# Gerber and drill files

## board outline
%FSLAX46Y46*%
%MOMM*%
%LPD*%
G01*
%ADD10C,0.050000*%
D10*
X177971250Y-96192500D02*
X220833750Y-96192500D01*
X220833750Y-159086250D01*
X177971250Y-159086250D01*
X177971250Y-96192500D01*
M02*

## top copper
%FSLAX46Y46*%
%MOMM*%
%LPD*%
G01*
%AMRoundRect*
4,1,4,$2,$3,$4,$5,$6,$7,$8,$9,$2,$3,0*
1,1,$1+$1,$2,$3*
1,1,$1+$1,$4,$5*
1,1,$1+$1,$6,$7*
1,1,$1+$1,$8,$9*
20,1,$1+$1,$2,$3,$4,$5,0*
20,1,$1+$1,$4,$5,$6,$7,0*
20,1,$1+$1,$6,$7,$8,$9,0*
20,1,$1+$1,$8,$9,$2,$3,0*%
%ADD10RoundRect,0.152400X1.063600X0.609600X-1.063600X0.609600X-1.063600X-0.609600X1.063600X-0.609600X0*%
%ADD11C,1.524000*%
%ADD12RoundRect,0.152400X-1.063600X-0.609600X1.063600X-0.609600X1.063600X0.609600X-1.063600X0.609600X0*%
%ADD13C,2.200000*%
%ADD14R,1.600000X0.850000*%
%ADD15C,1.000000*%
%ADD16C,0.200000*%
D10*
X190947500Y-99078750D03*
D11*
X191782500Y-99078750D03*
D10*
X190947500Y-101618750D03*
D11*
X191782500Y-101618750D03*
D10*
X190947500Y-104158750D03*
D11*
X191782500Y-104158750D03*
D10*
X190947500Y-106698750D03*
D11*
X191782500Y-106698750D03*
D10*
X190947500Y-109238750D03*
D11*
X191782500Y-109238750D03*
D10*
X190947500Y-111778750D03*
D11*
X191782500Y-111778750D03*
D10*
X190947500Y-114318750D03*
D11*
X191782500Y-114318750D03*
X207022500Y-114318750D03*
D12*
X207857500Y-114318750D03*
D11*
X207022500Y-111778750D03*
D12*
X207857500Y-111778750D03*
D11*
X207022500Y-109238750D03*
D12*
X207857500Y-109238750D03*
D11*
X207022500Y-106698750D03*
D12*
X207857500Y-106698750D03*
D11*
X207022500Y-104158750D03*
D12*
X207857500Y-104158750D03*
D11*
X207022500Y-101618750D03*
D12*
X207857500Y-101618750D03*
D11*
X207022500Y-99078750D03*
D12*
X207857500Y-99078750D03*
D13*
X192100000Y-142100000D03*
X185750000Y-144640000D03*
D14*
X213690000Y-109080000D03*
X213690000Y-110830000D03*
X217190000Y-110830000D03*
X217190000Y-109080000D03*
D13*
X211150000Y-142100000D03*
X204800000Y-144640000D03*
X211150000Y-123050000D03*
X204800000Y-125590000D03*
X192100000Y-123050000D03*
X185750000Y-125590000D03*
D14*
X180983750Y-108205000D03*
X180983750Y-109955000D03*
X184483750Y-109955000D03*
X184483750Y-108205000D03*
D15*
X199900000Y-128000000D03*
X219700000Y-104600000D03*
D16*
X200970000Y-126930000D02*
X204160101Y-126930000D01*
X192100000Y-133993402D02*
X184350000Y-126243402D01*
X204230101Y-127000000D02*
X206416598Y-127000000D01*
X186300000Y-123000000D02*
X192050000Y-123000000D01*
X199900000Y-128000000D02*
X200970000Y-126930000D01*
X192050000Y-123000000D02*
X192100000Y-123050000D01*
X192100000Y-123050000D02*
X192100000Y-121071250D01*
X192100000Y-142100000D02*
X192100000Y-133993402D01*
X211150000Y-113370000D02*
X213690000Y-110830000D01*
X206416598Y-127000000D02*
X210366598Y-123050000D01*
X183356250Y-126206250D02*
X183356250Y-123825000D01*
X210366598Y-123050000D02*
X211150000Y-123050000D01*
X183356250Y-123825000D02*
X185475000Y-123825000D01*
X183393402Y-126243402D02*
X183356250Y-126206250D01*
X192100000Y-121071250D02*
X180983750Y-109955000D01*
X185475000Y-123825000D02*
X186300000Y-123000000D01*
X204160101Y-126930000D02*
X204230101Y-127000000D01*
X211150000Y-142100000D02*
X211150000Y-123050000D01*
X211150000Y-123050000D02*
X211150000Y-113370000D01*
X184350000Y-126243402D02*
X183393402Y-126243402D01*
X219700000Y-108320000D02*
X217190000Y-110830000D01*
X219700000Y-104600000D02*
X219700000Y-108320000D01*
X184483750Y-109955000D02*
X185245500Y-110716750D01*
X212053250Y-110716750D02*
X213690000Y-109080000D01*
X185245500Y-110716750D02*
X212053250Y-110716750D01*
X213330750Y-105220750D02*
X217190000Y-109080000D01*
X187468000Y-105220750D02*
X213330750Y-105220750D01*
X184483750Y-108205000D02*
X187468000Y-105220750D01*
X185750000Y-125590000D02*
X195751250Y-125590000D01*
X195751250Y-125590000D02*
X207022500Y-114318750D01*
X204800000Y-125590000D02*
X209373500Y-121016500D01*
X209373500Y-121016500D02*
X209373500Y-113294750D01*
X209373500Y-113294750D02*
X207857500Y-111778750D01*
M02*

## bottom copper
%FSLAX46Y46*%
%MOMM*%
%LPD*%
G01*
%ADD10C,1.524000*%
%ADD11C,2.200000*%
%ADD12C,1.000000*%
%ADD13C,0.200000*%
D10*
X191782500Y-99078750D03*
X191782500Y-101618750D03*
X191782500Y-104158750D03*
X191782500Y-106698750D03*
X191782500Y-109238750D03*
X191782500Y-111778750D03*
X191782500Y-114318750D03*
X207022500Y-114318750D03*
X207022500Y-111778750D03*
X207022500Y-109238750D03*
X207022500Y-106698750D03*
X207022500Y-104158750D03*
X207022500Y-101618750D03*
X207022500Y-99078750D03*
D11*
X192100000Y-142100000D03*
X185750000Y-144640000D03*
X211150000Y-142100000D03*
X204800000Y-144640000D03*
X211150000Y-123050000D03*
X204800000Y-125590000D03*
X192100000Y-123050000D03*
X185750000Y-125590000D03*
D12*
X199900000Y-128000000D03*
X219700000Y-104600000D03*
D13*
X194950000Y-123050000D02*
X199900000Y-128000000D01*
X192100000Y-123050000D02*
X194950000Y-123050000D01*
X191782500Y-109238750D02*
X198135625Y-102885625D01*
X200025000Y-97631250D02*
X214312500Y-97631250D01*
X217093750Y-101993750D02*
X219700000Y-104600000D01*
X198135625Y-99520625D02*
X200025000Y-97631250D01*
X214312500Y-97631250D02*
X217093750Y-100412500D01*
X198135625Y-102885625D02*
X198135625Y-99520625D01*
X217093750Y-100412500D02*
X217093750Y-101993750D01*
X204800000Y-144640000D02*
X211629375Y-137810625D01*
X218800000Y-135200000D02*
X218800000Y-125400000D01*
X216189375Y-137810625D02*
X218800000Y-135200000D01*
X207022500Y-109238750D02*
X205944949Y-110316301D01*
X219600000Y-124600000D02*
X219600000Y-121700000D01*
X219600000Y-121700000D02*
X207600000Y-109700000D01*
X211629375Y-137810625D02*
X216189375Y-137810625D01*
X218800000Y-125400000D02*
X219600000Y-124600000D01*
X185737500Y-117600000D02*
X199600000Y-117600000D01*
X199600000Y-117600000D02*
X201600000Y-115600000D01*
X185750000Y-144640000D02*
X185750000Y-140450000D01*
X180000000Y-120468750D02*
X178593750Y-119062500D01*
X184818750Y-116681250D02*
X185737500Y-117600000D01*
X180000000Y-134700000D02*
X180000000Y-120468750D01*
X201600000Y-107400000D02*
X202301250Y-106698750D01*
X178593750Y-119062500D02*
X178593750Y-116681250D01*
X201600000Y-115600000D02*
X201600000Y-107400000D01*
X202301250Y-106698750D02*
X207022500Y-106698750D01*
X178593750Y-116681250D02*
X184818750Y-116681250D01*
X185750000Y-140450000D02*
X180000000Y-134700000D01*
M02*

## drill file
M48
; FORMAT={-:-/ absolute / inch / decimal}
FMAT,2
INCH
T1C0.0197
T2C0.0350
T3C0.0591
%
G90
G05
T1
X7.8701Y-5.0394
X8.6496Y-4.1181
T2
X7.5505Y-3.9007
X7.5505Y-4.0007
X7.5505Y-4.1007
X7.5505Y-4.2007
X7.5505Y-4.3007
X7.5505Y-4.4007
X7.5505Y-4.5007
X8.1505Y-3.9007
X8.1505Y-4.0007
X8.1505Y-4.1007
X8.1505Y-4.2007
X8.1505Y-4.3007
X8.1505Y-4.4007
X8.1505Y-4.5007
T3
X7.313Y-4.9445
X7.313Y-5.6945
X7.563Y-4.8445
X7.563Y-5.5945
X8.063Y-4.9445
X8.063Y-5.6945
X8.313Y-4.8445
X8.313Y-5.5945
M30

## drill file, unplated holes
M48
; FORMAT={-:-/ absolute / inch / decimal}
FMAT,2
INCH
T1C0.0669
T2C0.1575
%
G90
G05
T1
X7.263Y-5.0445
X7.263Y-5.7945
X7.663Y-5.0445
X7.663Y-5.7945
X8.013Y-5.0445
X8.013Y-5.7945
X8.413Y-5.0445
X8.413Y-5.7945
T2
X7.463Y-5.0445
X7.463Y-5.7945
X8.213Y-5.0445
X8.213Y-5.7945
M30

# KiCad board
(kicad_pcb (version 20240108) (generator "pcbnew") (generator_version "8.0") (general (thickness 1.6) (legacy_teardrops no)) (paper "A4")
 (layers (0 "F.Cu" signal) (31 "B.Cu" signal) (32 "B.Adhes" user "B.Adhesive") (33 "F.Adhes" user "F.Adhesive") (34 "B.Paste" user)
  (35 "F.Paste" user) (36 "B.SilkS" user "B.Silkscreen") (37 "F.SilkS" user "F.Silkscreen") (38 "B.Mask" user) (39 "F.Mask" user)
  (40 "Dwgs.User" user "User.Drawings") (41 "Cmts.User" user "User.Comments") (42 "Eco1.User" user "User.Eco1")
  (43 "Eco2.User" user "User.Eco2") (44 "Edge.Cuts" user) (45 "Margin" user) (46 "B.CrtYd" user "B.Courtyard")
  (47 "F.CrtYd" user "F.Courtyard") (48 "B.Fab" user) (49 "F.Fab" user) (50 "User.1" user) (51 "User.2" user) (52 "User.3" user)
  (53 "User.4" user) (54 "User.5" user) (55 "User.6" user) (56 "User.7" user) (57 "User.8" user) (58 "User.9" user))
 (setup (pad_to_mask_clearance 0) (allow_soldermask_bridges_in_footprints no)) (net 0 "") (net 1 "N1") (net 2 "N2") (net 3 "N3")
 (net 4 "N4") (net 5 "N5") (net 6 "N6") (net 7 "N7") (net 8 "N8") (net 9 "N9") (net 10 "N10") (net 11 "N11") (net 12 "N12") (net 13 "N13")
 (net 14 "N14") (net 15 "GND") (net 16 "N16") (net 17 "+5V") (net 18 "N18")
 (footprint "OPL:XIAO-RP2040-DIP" (layer "F.Cu") (at 199.4025 106.69875)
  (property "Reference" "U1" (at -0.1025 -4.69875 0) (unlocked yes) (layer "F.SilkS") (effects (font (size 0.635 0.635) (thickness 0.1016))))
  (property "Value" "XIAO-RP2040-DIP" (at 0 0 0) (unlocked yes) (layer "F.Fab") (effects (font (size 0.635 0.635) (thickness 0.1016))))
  (pad "1" smd roundrect (at -8.455 -7.62 180) (size 2.432 1.524) (layers "F.Cu" "F.Mask") (roundrect_rratio 0.1) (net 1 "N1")
   (thermal_bridge_angle 45))
  (pad "1" thru_hole circle (at -7.62 -7.62 180) (size 1.524 1.524) (drill 0.889) (layers "*.Cu" "*.Mask") (remove_unused_layers no)
   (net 1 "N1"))
  (pad "2" smd roundrect (at -8.455 -5.08 180) (size 2.432 1.524) (layers "F.Cu" "F.Mask") (roundrect_rratio 0.1) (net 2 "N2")
   (thermal_bridge_angle 45))
  (pad "2" thru_hole circle (at -7.62 -5.08 180) (size 1.524 1.524) (drill 0.889) (layers "*.Cu" "*.Mask") (remove_unused_layers no)
   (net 2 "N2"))
  (pad "3" smd roundrect (at -8.455 -2.54 180) (size 2.432 1.524) (layers "F.Cu" "F.Mask") (roundrect_rratio 0.1) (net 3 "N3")
   (thermal_bridge_angle 45))
  (pad "3" thru_hole circle (at -7.62 -2.54 180) (size 1.524 1.524) (drill 0.889) (layers "*.Cu" "*.Mask") (remove_unused_layers no)
   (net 3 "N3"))
  (pad "4" smd roundrect (at -8.455 0 180) (size 2.432 1.524) (layers "F.Cu" "F.Mask") (roundrect_rratio 0.1) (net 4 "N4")
   (thermal_bridge_angle 45))
  (pad "4" thru_hole circle (at -7.62 0 180) (size 1.524 1.524) (drill 0.889) (layers "*.Cu" "*.Mask") (remove_unused_layers no)
   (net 4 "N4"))
  (pad "5" smd roundrect (at -8.455 2.54 180) (size 2.432 1.524) (layers "F.Cu" "F.Mask") (roundrect_rratio 0.1) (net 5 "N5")
   (thermal_bridge_angle 45))
  (pad "5" thru_hole circle (at -7.62 2.54 180) (size 1.524 1.524) (drill 0.889) (layers "*.Cu" "*.Mask") (remove_unused_layers no)
   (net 5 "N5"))
  (pad "6" smd roundrect (at -8.455 5.08 180) (size 2.432 1.524) (layers "F.Cu" "F.Mask") (roundrect_rratio 0.1) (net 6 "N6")
   (thermal_bridge_angle 45))
  (pad "6" thru_hole circle (at -7.62 5.08 180) (size 1.524 1.524) (drill 0.889) (layers "*.Cu" "*.Mask") (remove_unused_layers no)
   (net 6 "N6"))
  (pad "7" smd roundrect (at -8.455 7.62 180) (size 2.432 1.524) (layers "F.Cu" "F.Mask") (roundrect_rratio 0.1) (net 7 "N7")
   (thermal_bridge_angle 45))
  (pad "7" thru_hole circle (at -7.62 7.62 180) (size 1.524 1.524) (drill 0.889) (layers "*.Cu" "*.Mask") (remove_unused_layers no)
   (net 7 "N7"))
  (pad "8" thru_hole circle (at 7.62 7.62) (size 1.524 1.524) (drill 0.889) (layers "*.Cu" "*.Mask") (remove_unused_layers no) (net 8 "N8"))
  (pad "8" smd roundrect (at 8.455 7.62) (size 2.432 1.524) (layers "F.Cu" "F.Mask") (roundrect_rratio 0.1) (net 8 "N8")
   (thermal_bridge_angle 45))
  (pad "9" thru_hole circle (at 7.62 5.08) (size 1.524 1.524) (drill 0.889) (layers "*.Cu" "*.Mask") (remove_unused_layers no) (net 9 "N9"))
  (pad "9" smd roundrect (at 8.455 5.08) (size 2.432 1.524) (layers "F.Cu" "F.Mask") (roundrect_rratio 0.1) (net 9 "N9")
   (thermal_bridge_angle 45))
  (pad "10" thru_hole circle (at 7.62 2.54) (size 1.524 1.524) (drill 0.889) (layers "*.Cu" "*.Mask") (remove_unused_layers no)
   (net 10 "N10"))
  (pad "10" smd roundrect (at 8.455 2.54) (size 2.432 1.524) (layers "F.Cu" "F.Mask") (roundrect_rratio 0.1) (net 10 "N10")
   (thermal_bridge_angle 45))
  (pad "11" thru_hole circle (at 7.62 0) (size 1.524 1.524) (drill 0.889) (layers "*.Cu" "*.Mask") (remove_unused_layers no) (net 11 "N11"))
  (pad "11" smd roundrect (at 8.455 0) (size 2.432 1.524) (layers "F.Cu" "F.Mask") (roundrect_rratio 0.1) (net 11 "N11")
   (thermal_bridge_angle 45))
  (pad "12" thru_hole circle (at 7.62 -2.54) (size 1.524 1.524) (drill 0.889) (layers "*.Cu" "*.Mask") (remove_unused_layers no)
   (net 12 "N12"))
  (pad "12" smd roundrect (at 8.455 -2.54) (size 2.432 1.524) (layers "F.Cu" "F.Mask") (roundrect_rratio 0.1) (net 12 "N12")
   (thermal_bridge_angle 45))
  (pad "13" thru_hole circle (at 7.62 -5.08) (size 1.524 1.524) (drill 0.889) (layers "*.Cu" "*.Mask") (remove_unused_layers no)
   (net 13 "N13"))
  (pad "13" smd roundrect (at 8.455 -5.08) (size 2.432 1.524) (layers "F.Cu" "F.Mask") (roundrect_rratio 0.1) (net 13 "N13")
   (thermal_bridge_angle 45))
  (pad "14" thru_hole circle (at 7.62 -7.62) (size 1.524 1.524) (drill 0.889) (layers "*.Cu" "*.Mask") (remove_unused_layers no)
   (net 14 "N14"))
  (pad "14" smd roundrect (at 8.455 -7.62) (size 2.432 1.524) (layers "F.Cu" "F.Mask") (roundrect_rratio 0.1) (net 14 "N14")
   (thermal_bridge_angle 45)))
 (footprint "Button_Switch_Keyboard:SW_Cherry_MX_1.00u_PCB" (layer "F.Cu") (at 192.1 142.1)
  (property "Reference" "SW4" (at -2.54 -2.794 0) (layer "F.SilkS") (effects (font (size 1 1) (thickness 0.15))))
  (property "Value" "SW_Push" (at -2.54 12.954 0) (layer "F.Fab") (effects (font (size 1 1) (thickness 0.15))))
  (pad "" np_thru_hole circle (at -7.62 5.08) (size 1.7 1.7) (drill 1.7) (layers "*.Cu" "*.Mask"))
  (pad "" np_thru_hole circle (at -2.54 5.08) (size 4 4) (drill 4) (layers "*.Cu" "*.Mask"))
  (pad "" np_thru_hole circle (at 2.54 5.08) (size 1.7 1.7) (drill 1.7) (layers "*.Cu" "*.Mask"))
  (pad "1" thru_hole circle (at 0 0) (size 2.2 2.2) (drill 1.5) (layers "*.Cu" "*.Mask") (remove_unused_layers no) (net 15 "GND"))
  (pad "2" thru_hole circle (at -6.35 2.54) (size 2.2 2.2) (drill 1.5) (layers "*.Cu" "*.Mask") (remove_unused_layers no) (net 11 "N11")))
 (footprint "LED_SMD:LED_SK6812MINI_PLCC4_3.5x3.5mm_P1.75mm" (layer "F.Cu") (at 215.44 109.955)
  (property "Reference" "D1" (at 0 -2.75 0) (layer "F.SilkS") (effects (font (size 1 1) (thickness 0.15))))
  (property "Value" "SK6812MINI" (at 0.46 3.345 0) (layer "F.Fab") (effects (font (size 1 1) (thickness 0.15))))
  (pad "1" smd rect (at -1.75 -0.875) (size 1.6 0.85) (layers "F.Cu" "F.Paste" "F.Mask") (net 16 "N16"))
  (pad "2" smd rect (at -1.75 0.875) (size 1.6 0.85) (layers "F.Cu" "F.Paste" "F.Mask") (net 15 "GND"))
  (pad "3" smd rect (at 1.75 0.875) (size 1.6 0.85) (layers "F.Cu" "F.Paste" "F.Mask") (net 5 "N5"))
  (pad "4" smd rect (at 1.75 -0.875) (size 1.6 0.85) (layers "F.Cu" "F.Paste" "F.Mask") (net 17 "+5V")))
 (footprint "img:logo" (layer "F.Cu") (at 215.554742 100.650524)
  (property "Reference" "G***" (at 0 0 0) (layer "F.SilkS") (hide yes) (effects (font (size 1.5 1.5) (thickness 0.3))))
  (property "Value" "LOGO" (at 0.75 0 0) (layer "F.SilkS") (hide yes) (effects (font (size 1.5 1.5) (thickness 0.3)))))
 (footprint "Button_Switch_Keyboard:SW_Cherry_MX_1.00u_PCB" (layer "F.Cu") (at 211.15 142.1)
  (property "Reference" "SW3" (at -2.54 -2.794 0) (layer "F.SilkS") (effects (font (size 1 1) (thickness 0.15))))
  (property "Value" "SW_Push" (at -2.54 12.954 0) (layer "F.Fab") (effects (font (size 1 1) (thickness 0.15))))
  (pad "" np_thru_hole circle (at -7.62 5.08) (size 1.7 1.7) (drill 1.7) (layers "*.Cu" "*.Mask"))
  (pad "" np_thru_hole circle (at -2.54 5.08) (size 4 4) (drill 4) (layers "*.Cu" "*.Mask"))
  (pad "" np_thru_hole circle (at 2.54 5.08) (size 1.7 1.7) (drill 1.7) (layers "*.Cu" "*.Mask"))
  (pad "1" thru_hole circle (at 0 0) (size 2.2 2.2) (drill 1.5) (layers "*.Cu" "*.Mask") (remove_unused_layers no) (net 15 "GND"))
  (pad "2" thru_hole circle (at -6.35 2.54) (size 2.2 2.2) (drill 1.5) (layers "*.Cu" "*.Mask") (remove_unused_layers no) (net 10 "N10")))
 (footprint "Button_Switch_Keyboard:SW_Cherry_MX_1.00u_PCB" (layer "F.Cu") (at 211.15 123.05)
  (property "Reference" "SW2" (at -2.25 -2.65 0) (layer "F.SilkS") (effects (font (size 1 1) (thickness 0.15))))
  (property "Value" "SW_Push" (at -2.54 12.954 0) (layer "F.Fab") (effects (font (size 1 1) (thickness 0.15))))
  (pad "" np_thru_hole circle (at -7.62 5.08) (size 1.7 1.7) (drill 1.7) (layers "*.Cu" "*.Mask"))
  (pad "" np_thru_hole circle (at -2.54 5.08) (size 4 4) (drill 4) (layers "*.Cu" "*.Mask"))
  (pad "" np_thru_hole circle (at 2.54 5.08) (size 1.7 1.7) (drill 1.7) (layers "*.Cu" "*.Mask"))
  (pad "1" thru_hole circle (at 0 0) (size 2.2 2.2) (drill 1.5) (layers "*.Cu" "*.Mask") (remove_unused_layers no) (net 15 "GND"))
  (pad "2" thru_hole circle (at -6.35 2.54) (size 2.2 2.2) (drill 1.5) (layers "*.Cu" "*.Mask") (remove_unused_layers no) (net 9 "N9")))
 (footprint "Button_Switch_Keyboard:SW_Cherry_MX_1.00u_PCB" (layer "F.Cu") (at 192.1 123.05)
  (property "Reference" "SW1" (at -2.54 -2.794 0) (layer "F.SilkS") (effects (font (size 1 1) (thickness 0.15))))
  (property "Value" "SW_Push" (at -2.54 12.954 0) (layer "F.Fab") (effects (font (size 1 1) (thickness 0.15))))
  (pad "" np_thru_hole circle (at -7.62 5.08) (size 1.7 1.7) (drill 1.7) (layers "*.Cu" "*.Mask"))
  (pad "" np_thru_hole circle (at -2.54 5.08) (size 4 4) (drill 4) (layers "*.Cu" "*.Mask"))
  (pad "" np_thru_hole circle (at 2.54 5.08) (size 1.7 1.7) (drill 1.7) (layers "*.Cu" "*.Mask"))
  (pad "1" thru_hole circle (at 0 0) (size 2.2 2.2) (drill 1.5) (layers "*.Cu" "*.Mask") (remove_unused_layers no) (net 15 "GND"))
  (pad "2" thru_hole circle (at -6.35 2.54) (size 2.2 2.2) (drill 1.5) (layers "*.Cu" "*.Mask") (remove_unused_layers no) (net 8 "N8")))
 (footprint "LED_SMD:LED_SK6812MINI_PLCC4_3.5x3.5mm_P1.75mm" (layer "F.Cu") (at 182.73375 109.08)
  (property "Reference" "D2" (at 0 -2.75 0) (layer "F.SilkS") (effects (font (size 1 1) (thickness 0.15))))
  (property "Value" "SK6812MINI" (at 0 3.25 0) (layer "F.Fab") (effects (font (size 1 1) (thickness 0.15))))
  (pad "1" smd rect (at -1.75 -0.875) (size 1.6 0.85) (layers "F.Cu" "F.Paste" "F.Mask") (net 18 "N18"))
  (pad "2" smd rect (at -1.75 0.875) (size 1.6 0.85) (layers "F.Cu" "F.Paste" "F.Mask") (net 15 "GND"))
  (pad "3" smd rect (at 1.75 0.875) (size 1.6 0.85) (layers "F.Cu" "F.Paste" "F.Mask") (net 16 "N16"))
  (pad "4" smd rect (at 1.75 -0.875) (size 1.6 0.85) (layers "F.Cu" "F.Paste" "F.Mask") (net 17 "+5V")))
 (gr_rect (start 177.97125 96.1925) (end 220.83375 159.08625) (stroke (width 0.05) (type default)) (fill none) (layer "Edge.Cuts"))
 (segment (start 200.97 126.93) (end 204.160101 126.93) (width 0.2) (layer "F.Cu") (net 15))
 (segment (start 192.1 133.993402) (end 184.35 126.243402) (width 0.2) (layer "F.Cu") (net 15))
 (segment (start 204.230101 127) (end 206.416598 127) (width 0.2) (layer "F.Cu") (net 15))
 (segment (start 186.3 123) (end 192.05 123) (width 0.2) (layer "F.Cu") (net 15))
 (segment (start 199.9 128) (end 200.97 126.93) (width 0.2) (layer "F.Cu") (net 15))
 (segment (start 192.05 123) (end 192.1 123.05) (width 0.2) (layer "F.Cu") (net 15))
 (segment (start 192.1 123.05) (end 192.1 121.07125) (width 0.2) (layer "F.Cu") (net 15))
 (segment (start 192.1 142.1) (end 192.1 133.993402) (width 0.2) (layer "F.Cu") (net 15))
 (segment (start 211.15 113.37) (end 213.69 110.83) (width 0.2) (layer "F.Cu") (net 15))
 (segment (start 206.416598 127) (end 210.366598 123.05) (width 0.2) (layer "F.Cu") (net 15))
 (segment (start 183.35625 126.20625) (end 183.35625 123.825) (width 0.2) (layer "F.Cu") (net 15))
 (segment (start 210.366598 123.05) (end 211.15 123.05) (width 0.2) (layer "F.Cu") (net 15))
 (segment (start 183.35625 123.825) (end 185.475 123.825) (width 0.2) (layer "F.Cu") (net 15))
 (segment (start 183.393402 126.243402) (end 183.35625 126.20625) (width 0.2) (layer "F.Cu") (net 15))
 (segment (start 192.1 121.07125) (end 180.98375 109.955) (width 0.2) (layer "F.Cu") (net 15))
 (segment (start 185.475 123.825) (end 186.3 123) (width 0.2) (layer "F.Cu") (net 15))
 (segment (start 204.160101 126.93) (end 204.230101 127) (width 0.2) (layer "F.Cu") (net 15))
 (segment (start 211.15 142.1) (end 211.15 123.05) (width 0.2) (layer "F.Cu") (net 15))
 (segment (start 211.15 123.05) (end 211.15 113.37) (width 0.2) (layer "F.Cu") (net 15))
 (segment (start 184.35 126.243402) (end 183.393402 126.243402) (width 0.2) (layer "F.Cu") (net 15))
 (via (at 199.9 128) (size 1) (drill 0.5) (layers "F.Cu" "B.Cu") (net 15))
 (segment (start 194.95 123.05) (end 199.9 128) (width 0.2) (layer "B.Cu") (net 15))
 (segment (start 192.1 123.05) (end 194.95 123.05) (width 0.2) (layer "B.Cu") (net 15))
 (segment (start 219.7 108.32) (end 217.19 110.83) (width 0.2) (layer "F.Cu") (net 5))
 (segment (start 219.7 104.6) (end 219.7 108.32) (width 0.2) (layer "F.Cu") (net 5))
 (via (at 219.7 104.6) (size 1) (drill 0.5) (layers "F.Cu" "B.Cu") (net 5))
 (segment (start 191.7825 109.23875) (end 198.135625 102.885625) (width 0.2) (layer "B.Cu") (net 5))
 (segment (start 200.025 97.63125) (end 214.3125 97.63125) (width 0.2) (layer "B.Cu") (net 5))
 (segment (start 217.09375 101.99375) (end 219.7 104.6) (width 0.2) (layer "B.Cu") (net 5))
 (segment (start 198.135625 99.520625) (end 200.025 97.63125) (width 0.2) (layer "B.Cu") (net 5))
 (segment (start 214.3125 97.63125) (end 217.09375 100.4125) (width 0.2) (layer "B.Cu") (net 5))
 (segment (start 198.135625 102.885625) (end 198.135625 99.520625) (width 0.2) (layer "B.Cu") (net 5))
 (segment (start 217.09375 100.4125) (end 217.09375 101.99375) (width 0.2) (layer "B.Cu") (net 5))
 (segment (start 184.48375 109.955) (end 185.2455 110.71675) (width 0.2) (layer "F.Cu") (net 16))
 (segment (start 212.05325 110.71675) (end 213.69 109.08) (width 0.2) (layer "F.Cu") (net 16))
 (segment (start 185.2455 110.71675) (end 212.05325 110.71675) (width 0.2) (layer "F.Cu") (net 16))
 (segment (start 213.33075 105.22075) (end 217.19 109.08) (width 0.2) (layer "F.Cu") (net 17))
 (segment (start 187.468 105.22075) (end 213.33075 105.22075) (width 0.2) (layer "F.Cu") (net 17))
 (segment (start 184.48375 108.205) (end 187.468 105.22075) (width 0.2) (layer "F.Cu") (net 17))
 (segment (start 185.75 125.59) (end 195.75125 125.59) (width 0.2) (layer "F.Cu") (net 8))
 (segment (start 195.75125 125.59) (end 207.0225 114.31875) (width 0.2) (layer "F.Cu") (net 8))
 (segment (start 204.8 125.59) (end 209.3735 121.0165) (width 0.2) (layer "F.Cu") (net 9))
 (segment (start 209.3735 121.0165) (end 209.3735 113.29475) (width 0.2) (layer "F.Cu") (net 9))
 (segment (start 209.3735 113.29475) (end 207.8575 111.77875) (width 0.2) (layer "F.Cu") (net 9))
 (segment (start 204.8 144.64) (end 211.629375 137.810625) (width 0.2) (layer "B.Cu") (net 10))
 (segment (start 218.8 135.2) (end 218.8 125.4) (width 0.2) (layer "B.Cu") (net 10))
 (segment (start 216.189375 137.810625) (end 218.8 135.2) (width 0.2) (layer "B.Cu") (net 10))
 (segment (start 207.0225 109.23875) (end 205.944949 110.316301) (width 0.2) (layer "B.Cu") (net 10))
 (segment (start 219.6 124.6) (end 219.6 121.7) (width 0.2) (layer "B.Cu") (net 10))
 (segment (start 219.6 121.7) (end 207.6 109.7) (width 0.2) (layer "B.Cu") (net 10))
 (segment (start 211.629375 137.810625) (end 216.189375 137.810625) (width 0.2) (layer "B.Cu") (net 10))
 (segment (start 218.8 125.4) (end 219.6 124.6) (width 0.2) (layer "B.Cu") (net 10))
 (segment (start 185.7375 117.6) (end 199.6 117.6) (width 0.2) (layer "B.Cu") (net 11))
 (segment (start 199.6 117.6) (end 201.6 115.6) (width 0.2) (layer "B.Cu") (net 11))
 (segment (start 185.75 144.64) (end 185.75 140.45) (width 0.2) (layer "B.Cu") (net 11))
 (segment (start 180 120.46875) (end 178.59375 119.0625) (width 0.2) (layer "B.Cu") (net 11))
 (segment (start 184.81875 116.68125) (end 185.7375 117.6) (width 0.2) (layer "B.Cu") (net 11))
 (segment (start 180 134.7) (end 180 120.46875) (width 0.2) (layer "B.Cu") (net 11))
 (segment (start 201.6 107.4) (end 202.30125 106.69875) (width 0.2) (layer "B.Cu") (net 11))
 (segment (start 178.59375 119.0625) (end 178.59375 116.68125) (width 0.2) (layer "B.Cu") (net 11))
 (segment (start 201.6 115.6) (end 201.6 107.4) (width 0.2) (layer "B.Cu") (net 11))
 (segment (start 202.30125 106.69875) (end 207.0225 106.69875) (width 0.2) (layer "B.Cu") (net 11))
 (segment (start 178.59375 116.68125) (end 184.81875 116.68125) (width 0.2) (layer "B.Cu") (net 11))
 (segment (start 185.75 140.45) (end 180 134.7) (width 0.2) (layer "B.Cu") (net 11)))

